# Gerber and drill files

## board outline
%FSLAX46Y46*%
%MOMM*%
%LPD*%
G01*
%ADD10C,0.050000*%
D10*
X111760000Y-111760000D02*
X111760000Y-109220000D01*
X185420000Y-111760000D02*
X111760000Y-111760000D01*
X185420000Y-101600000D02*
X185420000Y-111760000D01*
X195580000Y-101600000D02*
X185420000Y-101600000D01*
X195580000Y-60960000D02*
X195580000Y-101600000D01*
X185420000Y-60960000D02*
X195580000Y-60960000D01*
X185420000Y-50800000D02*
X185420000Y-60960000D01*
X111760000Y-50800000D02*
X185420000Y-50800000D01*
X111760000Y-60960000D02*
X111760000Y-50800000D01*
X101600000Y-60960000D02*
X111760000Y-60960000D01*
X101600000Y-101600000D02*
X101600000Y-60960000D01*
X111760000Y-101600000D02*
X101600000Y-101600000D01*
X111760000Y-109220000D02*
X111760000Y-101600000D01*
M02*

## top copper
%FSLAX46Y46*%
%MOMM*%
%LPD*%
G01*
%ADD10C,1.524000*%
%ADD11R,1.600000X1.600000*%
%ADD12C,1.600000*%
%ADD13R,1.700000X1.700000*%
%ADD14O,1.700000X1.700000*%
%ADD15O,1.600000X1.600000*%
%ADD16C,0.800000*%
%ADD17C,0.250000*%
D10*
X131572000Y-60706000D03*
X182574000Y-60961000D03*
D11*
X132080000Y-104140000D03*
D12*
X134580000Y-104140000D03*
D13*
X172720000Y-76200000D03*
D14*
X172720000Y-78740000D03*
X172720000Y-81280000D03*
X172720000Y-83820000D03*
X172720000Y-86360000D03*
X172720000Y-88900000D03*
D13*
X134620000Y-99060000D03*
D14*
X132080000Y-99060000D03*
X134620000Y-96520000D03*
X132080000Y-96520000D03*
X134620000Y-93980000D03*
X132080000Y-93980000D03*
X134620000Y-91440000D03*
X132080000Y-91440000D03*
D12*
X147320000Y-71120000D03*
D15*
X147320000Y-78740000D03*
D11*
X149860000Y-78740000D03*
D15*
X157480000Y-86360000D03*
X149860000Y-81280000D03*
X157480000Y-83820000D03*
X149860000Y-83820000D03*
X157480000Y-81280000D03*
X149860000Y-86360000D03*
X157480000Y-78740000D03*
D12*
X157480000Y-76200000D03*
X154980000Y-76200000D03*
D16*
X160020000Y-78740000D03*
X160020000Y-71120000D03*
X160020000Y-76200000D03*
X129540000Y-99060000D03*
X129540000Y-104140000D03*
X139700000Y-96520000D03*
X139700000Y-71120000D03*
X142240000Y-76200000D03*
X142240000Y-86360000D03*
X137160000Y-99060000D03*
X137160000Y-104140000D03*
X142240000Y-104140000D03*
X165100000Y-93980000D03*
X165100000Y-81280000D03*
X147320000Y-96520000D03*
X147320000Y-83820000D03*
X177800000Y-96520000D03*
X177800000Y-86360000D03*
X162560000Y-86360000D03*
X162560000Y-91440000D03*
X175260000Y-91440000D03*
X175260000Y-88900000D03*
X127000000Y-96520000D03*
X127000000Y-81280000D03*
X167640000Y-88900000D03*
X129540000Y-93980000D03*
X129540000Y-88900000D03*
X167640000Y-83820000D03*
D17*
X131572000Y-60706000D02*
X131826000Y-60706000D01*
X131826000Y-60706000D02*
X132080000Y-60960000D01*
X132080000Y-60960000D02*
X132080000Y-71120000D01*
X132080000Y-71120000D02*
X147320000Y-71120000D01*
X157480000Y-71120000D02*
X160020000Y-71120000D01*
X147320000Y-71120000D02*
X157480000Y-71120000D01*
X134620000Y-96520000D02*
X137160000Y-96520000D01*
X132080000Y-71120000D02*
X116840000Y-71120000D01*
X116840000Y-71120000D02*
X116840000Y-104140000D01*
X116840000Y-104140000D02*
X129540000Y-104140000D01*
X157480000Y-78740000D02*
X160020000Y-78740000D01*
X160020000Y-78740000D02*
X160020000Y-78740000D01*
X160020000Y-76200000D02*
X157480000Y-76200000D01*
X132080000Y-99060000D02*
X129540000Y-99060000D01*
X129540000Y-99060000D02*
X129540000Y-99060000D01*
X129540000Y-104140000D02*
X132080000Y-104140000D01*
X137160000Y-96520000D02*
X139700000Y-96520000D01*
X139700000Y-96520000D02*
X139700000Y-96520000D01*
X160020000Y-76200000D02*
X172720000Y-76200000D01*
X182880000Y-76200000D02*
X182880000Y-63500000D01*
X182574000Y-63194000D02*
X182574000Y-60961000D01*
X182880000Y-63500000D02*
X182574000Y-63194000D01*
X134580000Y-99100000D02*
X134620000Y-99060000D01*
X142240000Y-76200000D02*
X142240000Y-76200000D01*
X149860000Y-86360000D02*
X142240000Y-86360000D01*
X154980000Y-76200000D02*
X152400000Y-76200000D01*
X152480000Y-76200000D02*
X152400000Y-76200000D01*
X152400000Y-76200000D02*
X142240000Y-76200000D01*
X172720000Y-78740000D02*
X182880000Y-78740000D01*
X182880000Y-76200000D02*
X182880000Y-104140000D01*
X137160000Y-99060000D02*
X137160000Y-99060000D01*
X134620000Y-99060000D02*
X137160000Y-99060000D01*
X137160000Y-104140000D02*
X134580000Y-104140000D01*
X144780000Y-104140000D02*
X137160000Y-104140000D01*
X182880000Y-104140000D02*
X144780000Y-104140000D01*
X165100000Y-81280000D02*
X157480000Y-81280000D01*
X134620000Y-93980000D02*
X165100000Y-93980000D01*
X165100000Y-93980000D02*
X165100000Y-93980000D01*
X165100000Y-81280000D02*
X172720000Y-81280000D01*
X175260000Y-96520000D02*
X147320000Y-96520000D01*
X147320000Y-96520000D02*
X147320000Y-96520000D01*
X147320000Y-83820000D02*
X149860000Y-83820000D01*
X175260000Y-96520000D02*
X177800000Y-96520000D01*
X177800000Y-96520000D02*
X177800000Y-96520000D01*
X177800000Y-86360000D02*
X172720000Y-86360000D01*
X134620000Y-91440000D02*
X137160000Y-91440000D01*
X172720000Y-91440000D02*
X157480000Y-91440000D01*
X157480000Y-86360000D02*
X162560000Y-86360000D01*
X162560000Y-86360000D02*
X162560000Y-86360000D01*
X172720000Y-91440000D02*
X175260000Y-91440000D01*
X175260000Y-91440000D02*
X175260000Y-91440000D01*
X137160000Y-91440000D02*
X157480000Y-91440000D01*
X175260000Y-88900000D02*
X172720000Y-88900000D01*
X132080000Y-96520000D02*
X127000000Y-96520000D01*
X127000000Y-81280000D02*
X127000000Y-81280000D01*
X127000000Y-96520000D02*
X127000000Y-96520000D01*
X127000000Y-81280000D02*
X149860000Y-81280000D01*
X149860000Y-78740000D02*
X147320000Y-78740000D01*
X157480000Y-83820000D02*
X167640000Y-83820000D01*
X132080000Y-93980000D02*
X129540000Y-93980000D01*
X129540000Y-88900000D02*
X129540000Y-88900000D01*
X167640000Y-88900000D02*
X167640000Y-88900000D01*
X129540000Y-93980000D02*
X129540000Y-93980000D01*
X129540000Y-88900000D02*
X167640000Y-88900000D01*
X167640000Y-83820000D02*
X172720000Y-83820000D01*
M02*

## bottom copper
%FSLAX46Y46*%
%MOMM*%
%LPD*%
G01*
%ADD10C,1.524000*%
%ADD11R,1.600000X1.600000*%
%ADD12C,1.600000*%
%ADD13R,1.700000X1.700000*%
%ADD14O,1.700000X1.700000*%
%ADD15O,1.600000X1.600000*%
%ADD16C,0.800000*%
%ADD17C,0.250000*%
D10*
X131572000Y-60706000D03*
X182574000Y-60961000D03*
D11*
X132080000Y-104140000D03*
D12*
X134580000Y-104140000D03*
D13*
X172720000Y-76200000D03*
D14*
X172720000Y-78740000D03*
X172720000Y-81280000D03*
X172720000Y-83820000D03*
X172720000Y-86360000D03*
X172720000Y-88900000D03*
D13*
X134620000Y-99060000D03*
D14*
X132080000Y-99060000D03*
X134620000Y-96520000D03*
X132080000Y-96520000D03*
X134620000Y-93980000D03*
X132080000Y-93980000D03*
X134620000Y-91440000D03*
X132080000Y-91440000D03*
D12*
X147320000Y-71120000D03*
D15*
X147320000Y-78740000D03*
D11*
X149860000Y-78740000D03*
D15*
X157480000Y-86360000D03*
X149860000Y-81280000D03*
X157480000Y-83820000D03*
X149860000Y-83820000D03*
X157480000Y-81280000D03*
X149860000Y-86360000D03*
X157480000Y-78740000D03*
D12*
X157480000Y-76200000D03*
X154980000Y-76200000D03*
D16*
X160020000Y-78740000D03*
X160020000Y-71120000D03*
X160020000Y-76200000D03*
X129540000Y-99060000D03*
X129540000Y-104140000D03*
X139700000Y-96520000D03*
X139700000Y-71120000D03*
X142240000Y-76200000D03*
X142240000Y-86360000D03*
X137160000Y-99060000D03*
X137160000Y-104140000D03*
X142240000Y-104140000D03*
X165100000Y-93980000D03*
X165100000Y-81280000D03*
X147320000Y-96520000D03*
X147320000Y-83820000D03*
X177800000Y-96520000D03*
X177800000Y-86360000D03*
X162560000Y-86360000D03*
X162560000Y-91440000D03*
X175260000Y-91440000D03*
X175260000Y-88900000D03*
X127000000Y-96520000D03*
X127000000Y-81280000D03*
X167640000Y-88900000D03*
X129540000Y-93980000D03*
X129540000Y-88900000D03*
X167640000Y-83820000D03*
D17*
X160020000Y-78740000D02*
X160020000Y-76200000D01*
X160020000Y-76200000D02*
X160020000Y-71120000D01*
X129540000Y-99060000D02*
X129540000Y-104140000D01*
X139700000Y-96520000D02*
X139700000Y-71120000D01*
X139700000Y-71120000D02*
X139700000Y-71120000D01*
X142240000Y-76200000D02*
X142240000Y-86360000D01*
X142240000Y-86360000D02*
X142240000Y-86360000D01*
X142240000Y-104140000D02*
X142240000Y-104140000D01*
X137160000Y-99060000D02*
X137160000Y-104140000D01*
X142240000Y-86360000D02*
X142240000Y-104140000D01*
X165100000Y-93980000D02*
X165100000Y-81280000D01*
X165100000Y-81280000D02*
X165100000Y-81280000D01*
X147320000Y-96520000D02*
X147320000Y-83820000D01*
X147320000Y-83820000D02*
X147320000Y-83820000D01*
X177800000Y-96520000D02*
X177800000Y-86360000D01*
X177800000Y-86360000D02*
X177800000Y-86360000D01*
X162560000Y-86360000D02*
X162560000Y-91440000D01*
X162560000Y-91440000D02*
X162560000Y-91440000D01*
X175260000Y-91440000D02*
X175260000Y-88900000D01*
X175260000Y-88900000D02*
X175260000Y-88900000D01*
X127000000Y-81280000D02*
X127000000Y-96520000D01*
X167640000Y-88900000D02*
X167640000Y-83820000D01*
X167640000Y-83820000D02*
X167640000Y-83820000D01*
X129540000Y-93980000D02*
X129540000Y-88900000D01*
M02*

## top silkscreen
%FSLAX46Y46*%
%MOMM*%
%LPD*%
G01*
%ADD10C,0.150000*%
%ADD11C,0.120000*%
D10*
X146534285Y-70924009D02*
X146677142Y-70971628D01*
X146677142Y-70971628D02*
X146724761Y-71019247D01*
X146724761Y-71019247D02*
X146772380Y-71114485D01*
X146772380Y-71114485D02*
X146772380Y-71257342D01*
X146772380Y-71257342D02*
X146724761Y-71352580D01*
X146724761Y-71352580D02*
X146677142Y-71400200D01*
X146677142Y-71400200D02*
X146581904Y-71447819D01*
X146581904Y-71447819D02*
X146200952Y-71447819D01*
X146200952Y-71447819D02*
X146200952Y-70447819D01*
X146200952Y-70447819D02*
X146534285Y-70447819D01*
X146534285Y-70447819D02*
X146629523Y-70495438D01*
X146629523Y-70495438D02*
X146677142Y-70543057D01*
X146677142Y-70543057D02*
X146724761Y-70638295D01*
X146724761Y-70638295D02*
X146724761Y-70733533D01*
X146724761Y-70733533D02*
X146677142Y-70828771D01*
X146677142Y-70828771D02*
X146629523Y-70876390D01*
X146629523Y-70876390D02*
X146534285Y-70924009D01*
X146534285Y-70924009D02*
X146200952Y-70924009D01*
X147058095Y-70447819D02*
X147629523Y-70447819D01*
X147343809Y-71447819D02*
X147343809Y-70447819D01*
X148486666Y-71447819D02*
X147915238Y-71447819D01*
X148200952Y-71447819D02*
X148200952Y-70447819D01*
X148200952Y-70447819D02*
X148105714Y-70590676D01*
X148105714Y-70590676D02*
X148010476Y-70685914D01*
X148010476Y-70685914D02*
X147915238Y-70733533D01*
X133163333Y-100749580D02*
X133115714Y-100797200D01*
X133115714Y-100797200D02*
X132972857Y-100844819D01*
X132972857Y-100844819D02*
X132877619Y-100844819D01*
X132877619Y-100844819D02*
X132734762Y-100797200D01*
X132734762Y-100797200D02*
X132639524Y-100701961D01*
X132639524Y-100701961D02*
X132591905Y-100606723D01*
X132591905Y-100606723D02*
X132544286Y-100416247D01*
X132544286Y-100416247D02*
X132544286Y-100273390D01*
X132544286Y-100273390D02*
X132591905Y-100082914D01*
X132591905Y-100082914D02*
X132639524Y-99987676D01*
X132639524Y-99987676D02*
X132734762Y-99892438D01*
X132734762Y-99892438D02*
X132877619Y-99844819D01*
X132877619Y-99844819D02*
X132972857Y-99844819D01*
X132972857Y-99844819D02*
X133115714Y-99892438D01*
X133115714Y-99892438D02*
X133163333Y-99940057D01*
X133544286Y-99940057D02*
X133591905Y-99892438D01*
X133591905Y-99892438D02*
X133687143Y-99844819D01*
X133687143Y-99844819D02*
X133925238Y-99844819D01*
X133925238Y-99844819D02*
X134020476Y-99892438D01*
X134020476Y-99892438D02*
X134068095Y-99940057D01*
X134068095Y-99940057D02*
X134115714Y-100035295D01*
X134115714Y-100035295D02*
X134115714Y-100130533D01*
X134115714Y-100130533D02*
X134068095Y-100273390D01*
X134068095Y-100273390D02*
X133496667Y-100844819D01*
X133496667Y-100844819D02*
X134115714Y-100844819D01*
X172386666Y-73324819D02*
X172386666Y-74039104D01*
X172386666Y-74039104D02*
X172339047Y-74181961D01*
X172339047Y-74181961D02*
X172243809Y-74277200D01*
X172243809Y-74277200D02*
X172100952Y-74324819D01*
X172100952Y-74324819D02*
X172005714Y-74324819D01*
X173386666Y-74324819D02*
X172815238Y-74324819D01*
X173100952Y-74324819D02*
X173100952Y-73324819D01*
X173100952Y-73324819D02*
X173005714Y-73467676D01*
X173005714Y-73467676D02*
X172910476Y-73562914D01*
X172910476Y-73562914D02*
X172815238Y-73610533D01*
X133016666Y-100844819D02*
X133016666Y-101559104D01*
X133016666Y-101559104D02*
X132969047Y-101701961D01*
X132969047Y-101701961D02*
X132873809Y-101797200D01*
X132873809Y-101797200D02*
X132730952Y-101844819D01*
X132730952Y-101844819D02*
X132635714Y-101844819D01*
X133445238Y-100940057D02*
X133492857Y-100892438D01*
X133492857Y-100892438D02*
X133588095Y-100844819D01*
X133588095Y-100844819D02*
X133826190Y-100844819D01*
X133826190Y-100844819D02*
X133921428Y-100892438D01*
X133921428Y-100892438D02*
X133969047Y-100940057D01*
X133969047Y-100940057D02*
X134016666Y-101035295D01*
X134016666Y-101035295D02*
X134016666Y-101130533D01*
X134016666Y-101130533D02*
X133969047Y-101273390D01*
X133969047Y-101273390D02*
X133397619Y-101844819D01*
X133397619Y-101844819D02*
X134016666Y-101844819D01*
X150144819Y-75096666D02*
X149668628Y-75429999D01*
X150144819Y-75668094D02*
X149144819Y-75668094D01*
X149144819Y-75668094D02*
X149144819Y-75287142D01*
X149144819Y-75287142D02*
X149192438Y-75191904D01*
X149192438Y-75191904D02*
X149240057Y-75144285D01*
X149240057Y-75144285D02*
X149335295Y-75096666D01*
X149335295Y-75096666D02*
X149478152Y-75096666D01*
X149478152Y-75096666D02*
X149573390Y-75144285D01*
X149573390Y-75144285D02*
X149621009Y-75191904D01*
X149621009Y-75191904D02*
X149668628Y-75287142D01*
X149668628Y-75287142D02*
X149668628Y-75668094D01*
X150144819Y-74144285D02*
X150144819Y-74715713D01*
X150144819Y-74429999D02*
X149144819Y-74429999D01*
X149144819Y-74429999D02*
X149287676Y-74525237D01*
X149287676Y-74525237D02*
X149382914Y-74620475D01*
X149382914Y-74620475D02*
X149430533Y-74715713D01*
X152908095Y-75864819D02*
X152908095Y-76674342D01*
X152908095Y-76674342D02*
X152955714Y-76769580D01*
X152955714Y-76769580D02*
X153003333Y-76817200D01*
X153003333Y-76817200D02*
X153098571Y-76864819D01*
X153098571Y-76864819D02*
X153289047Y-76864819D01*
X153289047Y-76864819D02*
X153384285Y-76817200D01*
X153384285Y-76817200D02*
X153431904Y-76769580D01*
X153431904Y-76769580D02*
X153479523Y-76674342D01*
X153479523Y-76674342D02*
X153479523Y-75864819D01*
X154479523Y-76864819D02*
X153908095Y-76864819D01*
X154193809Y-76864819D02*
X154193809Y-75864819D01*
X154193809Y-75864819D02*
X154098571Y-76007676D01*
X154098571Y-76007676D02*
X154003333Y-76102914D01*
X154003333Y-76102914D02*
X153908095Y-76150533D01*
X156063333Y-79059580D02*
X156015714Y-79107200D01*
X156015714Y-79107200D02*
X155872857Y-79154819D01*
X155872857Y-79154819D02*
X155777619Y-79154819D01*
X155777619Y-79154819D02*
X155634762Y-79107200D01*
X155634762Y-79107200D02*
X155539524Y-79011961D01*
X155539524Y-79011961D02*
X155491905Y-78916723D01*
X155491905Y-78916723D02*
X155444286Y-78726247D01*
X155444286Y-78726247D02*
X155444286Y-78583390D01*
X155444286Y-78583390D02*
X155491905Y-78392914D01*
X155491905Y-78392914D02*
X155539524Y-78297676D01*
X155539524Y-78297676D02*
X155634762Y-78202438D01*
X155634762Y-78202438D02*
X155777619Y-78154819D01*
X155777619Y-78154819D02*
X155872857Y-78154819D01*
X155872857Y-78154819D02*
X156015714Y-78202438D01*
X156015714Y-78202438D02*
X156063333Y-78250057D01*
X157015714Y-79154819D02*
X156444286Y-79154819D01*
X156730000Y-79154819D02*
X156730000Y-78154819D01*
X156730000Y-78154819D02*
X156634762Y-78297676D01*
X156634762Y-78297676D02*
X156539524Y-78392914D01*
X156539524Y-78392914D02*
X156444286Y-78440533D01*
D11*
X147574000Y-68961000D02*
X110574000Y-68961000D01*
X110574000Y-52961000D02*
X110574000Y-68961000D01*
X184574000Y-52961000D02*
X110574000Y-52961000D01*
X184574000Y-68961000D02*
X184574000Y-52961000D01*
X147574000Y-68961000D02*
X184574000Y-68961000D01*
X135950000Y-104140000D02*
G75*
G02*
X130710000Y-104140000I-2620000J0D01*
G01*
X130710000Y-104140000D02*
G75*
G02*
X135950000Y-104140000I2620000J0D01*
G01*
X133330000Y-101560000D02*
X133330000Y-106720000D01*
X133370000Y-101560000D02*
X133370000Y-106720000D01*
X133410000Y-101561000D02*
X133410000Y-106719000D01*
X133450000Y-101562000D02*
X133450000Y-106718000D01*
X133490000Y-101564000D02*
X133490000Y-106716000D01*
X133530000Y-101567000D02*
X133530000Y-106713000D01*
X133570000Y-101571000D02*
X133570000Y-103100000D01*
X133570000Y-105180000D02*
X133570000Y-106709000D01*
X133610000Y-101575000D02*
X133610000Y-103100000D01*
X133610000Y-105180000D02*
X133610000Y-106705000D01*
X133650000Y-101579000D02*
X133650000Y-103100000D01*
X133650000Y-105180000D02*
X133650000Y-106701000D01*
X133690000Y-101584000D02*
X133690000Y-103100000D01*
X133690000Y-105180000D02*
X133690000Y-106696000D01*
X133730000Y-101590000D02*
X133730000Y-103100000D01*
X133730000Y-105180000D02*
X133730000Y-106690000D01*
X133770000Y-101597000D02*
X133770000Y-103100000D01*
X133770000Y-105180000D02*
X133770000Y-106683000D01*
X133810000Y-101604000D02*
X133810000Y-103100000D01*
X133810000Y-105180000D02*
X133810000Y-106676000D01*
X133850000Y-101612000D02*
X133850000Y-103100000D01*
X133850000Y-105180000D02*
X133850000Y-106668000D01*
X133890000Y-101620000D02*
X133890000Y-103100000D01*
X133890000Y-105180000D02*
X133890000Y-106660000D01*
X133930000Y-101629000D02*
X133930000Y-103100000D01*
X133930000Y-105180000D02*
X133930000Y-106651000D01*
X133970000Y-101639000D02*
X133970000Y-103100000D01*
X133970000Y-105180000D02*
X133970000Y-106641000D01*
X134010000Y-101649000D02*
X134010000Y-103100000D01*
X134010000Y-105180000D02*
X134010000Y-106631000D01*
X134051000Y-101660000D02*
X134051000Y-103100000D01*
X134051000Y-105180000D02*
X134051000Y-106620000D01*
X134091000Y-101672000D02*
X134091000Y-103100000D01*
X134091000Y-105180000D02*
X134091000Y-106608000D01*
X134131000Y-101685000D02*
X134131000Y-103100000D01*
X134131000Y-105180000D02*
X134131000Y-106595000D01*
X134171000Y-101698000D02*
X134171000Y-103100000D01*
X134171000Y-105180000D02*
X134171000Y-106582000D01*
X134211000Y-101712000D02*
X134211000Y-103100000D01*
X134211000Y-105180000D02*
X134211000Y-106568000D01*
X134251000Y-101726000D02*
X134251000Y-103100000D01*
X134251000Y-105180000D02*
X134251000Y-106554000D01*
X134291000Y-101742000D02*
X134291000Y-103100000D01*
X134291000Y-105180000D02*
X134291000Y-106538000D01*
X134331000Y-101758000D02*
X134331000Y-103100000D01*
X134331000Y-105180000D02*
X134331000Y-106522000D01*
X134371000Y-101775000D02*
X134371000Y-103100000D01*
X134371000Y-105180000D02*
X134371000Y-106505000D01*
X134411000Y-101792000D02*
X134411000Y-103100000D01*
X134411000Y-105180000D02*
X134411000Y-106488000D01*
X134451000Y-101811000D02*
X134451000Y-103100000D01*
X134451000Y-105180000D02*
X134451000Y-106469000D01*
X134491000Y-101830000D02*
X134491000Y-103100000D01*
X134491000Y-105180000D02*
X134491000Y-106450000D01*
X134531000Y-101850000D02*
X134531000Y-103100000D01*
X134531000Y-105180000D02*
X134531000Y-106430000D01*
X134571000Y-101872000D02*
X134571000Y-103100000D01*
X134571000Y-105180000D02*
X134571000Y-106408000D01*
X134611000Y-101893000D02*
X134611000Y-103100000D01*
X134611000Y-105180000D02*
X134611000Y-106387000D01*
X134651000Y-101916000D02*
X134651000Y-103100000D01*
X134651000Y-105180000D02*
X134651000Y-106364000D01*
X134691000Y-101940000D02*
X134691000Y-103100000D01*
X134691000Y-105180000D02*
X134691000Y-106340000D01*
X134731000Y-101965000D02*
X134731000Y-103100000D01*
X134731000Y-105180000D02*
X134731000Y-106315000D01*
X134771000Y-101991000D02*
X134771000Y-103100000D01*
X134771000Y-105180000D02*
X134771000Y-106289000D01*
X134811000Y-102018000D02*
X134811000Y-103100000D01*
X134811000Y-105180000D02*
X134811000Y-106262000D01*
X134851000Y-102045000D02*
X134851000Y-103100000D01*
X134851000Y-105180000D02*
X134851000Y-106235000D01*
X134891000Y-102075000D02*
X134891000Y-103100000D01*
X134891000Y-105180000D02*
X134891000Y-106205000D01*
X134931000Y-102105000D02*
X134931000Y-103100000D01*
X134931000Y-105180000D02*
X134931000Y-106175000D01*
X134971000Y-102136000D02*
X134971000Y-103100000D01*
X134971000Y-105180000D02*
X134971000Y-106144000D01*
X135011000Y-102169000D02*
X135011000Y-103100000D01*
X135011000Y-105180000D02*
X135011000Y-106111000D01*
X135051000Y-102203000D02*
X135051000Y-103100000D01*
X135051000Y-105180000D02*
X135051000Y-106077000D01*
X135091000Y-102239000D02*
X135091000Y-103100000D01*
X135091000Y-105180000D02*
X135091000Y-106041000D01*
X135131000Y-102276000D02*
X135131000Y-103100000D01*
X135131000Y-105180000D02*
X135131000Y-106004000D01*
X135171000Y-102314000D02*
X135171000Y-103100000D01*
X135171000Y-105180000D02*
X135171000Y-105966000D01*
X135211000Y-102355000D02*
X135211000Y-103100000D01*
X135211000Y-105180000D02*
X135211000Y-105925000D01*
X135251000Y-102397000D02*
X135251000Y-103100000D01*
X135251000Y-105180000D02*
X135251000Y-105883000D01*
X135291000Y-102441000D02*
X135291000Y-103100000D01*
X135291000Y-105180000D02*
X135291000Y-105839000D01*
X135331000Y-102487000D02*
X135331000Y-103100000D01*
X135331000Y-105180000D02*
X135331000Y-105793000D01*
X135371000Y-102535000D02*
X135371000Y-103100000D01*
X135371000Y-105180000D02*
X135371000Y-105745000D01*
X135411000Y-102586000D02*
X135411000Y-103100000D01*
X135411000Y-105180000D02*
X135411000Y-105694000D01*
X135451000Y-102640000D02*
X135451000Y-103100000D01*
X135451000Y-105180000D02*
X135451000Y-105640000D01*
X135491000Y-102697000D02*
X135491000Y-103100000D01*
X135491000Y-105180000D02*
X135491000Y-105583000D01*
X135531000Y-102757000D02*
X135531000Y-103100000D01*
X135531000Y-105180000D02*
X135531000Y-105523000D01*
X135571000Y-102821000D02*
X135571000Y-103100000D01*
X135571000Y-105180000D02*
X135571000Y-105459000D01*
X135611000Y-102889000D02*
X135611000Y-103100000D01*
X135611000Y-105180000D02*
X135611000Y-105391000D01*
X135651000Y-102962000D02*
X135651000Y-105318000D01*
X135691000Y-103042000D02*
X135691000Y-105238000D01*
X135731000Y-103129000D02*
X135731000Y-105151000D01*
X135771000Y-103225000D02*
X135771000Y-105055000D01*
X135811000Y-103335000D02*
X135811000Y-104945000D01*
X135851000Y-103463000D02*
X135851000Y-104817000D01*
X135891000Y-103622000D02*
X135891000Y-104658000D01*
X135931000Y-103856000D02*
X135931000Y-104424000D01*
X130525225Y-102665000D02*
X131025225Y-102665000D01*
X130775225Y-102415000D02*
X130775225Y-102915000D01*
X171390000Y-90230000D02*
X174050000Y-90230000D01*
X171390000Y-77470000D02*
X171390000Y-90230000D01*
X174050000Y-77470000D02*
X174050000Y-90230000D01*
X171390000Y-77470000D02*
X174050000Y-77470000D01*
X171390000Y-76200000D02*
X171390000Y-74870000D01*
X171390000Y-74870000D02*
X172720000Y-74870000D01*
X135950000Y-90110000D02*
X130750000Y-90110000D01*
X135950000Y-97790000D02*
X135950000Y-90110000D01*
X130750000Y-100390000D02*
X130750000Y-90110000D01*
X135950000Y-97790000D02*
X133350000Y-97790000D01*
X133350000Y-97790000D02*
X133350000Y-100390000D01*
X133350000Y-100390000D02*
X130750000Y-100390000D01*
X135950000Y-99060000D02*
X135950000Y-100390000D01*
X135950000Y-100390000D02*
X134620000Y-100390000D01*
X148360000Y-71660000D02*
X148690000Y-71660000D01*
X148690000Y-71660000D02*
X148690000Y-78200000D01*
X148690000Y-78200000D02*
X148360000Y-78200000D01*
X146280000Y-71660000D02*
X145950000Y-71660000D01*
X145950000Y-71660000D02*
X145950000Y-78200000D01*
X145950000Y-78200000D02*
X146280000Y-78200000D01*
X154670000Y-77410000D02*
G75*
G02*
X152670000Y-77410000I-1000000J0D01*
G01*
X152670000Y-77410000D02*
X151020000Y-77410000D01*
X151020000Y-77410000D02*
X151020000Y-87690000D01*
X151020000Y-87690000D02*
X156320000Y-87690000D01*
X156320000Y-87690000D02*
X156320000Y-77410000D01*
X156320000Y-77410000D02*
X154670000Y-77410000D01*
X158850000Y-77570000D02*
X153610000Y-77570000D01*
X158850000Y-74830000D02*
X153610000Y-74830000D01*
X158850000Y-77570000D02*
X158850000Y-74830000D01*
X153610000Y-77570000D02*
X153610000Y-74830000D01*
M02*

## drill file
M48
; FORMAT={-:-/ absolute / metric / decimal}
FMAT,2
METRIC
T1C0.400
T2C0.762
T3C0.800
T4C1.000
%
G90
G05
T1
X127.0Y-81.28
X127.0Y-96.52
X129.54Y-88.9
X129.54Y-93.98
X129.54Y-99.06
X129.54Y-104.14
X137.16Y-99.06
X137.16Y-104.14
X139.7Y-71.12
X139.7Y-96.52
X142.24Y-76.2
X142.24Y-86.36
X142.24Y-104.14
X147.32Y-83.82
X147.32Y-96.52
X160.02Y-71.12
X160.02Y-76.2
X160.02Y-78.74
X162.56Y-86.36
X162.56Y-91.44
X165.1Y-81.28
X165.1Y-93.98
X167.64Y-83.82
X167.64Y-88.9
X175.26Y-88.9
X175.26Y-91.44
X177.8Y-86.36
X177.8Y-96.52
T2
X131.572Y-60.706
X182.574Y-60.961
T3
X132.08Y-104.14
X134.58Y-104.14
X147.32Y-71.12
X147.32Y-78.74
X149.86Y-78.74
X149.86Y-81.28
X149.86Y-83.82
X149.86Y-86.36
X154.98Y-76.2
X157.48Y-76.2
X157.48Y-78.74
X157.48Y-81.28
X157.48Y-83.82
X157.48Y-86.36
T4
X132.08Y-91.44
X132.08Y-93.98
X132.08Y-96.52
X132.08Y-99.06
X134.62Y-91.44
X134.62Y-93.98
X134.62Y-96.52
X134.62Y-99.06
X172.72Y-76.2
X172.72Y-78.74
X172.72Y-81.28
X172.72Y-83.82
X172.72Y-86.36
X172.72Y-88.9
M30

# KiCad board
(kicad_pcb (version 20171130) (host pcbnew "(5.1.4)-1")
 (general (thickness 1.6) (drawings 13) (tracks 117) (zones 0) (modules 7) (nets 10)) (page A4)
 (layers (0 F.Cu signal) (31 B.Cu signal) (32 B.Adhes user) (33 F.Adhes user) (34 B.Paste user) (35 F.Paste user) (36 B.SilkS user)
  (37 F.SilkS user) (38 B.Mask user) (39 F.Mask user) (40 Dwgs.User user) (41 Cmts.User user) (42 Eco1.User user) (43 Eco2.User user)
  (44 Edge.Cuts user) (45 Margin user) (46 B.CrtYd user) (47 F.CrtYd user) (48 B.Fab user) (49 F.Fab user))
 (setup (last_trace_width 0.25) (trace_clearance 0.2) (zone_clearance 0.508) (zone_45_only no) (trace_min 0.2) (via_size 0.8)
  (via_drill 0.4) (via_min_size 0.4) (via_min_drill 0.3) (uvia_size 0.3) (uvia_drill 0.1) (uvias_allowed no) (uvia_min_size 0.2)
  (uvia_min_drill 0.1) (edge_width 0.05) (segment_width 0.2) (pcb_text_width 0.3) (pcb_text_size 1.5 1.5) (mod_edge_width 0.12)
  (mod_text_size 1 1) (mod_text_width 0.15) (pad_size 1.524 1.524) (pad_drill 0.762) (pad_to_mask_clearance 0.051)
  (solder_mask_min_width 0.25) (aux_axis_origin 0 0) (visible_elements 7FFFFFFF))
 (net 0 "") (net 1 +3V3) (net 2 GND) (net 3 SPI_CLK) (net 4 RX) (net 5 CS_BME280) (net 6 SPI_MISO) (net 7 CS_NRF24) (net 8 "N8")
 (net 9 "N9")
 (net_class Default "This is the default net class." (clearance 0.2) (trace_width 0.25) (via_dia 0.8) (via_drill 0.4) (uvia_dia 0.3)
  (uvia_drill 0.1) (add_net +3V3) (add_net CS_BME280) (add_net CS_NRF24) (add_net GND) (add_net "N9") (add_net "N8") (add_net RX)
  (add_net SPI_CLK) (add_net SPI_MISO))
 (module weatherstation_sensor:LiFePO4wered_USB (layer F.Cu) (at 147.32 60.96 180)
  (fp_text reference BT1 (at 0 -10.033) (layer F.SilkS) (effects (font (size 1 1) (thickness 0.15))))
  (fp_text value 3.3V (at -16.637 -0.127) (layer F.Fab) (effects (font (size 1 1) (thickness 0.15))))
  (fp_line (start -0.254 -8.001) (end 36.746 -8.001) (layer F.SilkS) (width 0.12))
  (fp_line (start 36.746 7.999) (end 36.746 -8.001) (layer F.SilkS) (width 0.12))
  (fp_line (start -37.254 7.999) (end 36.746 7.999) (layer F.SilkS) (width 0.12))
  (fp_line (start -37.254 -8.001) (end -37.254 7.999) (layer F.SilkS) (width 0.12))
  (fp_line (start -0.254 -8.001) (end -37.254 -8.001) (layer F.SilkS) (width 0.12))
  (pad 1 thru_hole circle (at 15.748 0.254 180) (size 1.524 1.524) (drill 0.762) (layers *.Cu *.Mask) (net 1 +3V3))
  (pad 2 thru_hole circle (at -35.254 -0.001 180) (size 1.524 1.524) (drill 0.762) (layers *.Cu *.Mask) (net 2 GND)))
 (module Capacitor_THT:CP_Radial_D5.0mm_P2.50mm (layer F.Cu) (at 132.08 104.14)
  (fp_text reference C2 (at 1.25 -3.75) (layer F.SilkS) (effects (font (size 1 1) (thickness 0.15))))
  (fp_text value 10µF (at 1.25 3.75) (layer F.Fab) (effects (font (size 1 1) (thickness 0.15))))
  (fp_circle (center 1.25 0) (end 3.87 0) (layer F.SilkS) (width 0.12))
  (fp_line (start 1.25 -2.58) (end 1.25 2.58) (layer F.SilkS) (width 0.12))
  (fp_line (start 1.29 -2.58) (end 1.29 2.58) (layer F.SilkS) (width 0.12))
  (fp_line (start 1.33 -2.579) (end 1.33 2.579) (layer F.SilkS) (width 0.12))
  (fp_line (start 1.37 -2.578) (end 1.37 2.578) (layer F.SilkS) (width 0.12))
  (fp_line (start 1.41 -2.576) (end 1.41 2.576) (layer F.SilkS) (width 0.12))
  (fp_line (start 1.45 -2.573) (end 1.45 2.573) (layer F.SilkS) (width 0.12))
  (fp_line (start 1.49 -2.569) (end 1.49 -1.04) (layer F.SilkS) (width 0.12))
  (fp_line (start 1.49 1.04) (end 1.49 2.569) (layer F.SilkS) (width 0.12))
  (fp_line (start 1.53 -2.565) (end 1.53 -1.04) (layer F.SilkS) (width 0.12))
  (fp_line (start 1.53 1.04) (end 1.53 2.565) (layer F.SilkS) (width 0.12))
  (fp_line (start 1.57 -2.561) (end 1.57 -1.04) (layer F.SilkS) (width 0.12))
  (fp_line (start 1.57 1.04) (end 1.57 2.561) (layer F.SilkS) (width 0.12))
  (fp_line (start 1.61 -2.556) (end 1.61 -1.04) (layer F.SilkS) (width 0.12))
  (fp_line (start 1.61 1.04) (end 1.61 2.556) (layer F.SilkS) (width 0.12))
  (fp_line (start 1.65 -2.55) (end 1.65 -1.04) (layer F.SilkS) (width 0.12))
  (fp_line (start 1.65 1.04) (end 1.65 2.55) (layer F.SilkS) (width 0.12))
  (fp_line (start 1.69 -2.543) (end 1.69 -1.04) (layer F.SilkS) (width 0.12))
  (fp_line (start 1.69 1.04) (end 1.69 2.543) (layer F.SilkS) (width 0.12))
  (fp_line (start 1.73 -2.536) (end 1.73 -1.04) (layer F.SilkS) (width 0.12))
  (fp_line (start 1.73 1.04) (end 1.73 2.536) (layer F.SilkS) (width 0.12))
  (fp_line (start 1.77 -2.528) (end 1.77 -1.04) (layer F.SilkS) (width 0.12))
  (fp_line (start 1.77 1.04) (end 1.77 2.528) (layer F.SilkS) (width 0.12))
  (fp_line (start 1.81 -2.52) (end 1.81 -1.04) (layer F.SilkS) (width 0.12))
  (fp_line (start 1.81 1.04) (end 1.81 2.52) (layer F.SilkS) (width 0.12))
  (fp_line (start 1.85 -2.511) (end 1.85 -1.04) (layer F.SilkS) (width 0.12))
  (fp_line (start 1.85 1.04) (end 1.85 2.511) (layer F.SilkS) (width 0.12))
  (fp_line (start 1.89 -2.501) (end 1.89 -1.04) (layer F.SilkS) (width 0.12))
  (fp_line (start 1.89 1.04) (end 1.89 2.501) (layer F.SilkS) (width 0.12))
  (fp_line (start 1.93 -2.491) (end 1.93 -1.04) (layer F.SilkS) (width 0.12))
  (fp_line (start 1.93 1.04) (end 1.93 2.491) (layer F.SilkS) (width 0.12))
  (fp_line (start 1.971 -2.48) (end 1.971 -1.04) (layer F.SilkS) (width 0.12))
  (fp_line (start 1.971 1.04) (end 1.971 2.48) (layer F.SilkS) (width 0.12))
  (fp_line (start 2.011 -2.468) (end 2.011 -1.04) (layer F.SilkS) (width 0.12))
  (fp_line (start 2.011 1.04) (end 2.011 2.468) (layer F.SilkS) (width 0.12))
  (fp_line (start 2.051 -2.455) (end 2.051 -1.04) (layer F.SilkS) (width 0.12))
  (fp_line (start 2.051 1.04) (end 2.051 2.455) (layer F.SilkS) (width 0.12))
  (fp_line (start 2.091 -2.442) (end 2.091 -1.04) (layer F.SilkS) (width 0.12))
  (fp_line (start 2.091 1.04) (end 2.091 2.442) (layer F.SilkS) (width 0.12))
  (fp_line (start 2.131 -2.428) (end 2.131 -1.04) (layer F.SilkS) (width 0.12))
  (fp_line (start 2.131 1.04) (end 2.131 2.428) (layer F.SilkS) (width 0.12))
  (fp_line (start 2.171 -2.414) (end 2.171 -1.04) (layer F.SilkS) (width 0.12))
  (fp_line (start 2.171 1.04) (end 2.171 2.414) (layer F.SilkS) (width 0.12))
  (fp_line (start 2.211 -2.398) (end 2.211 -1.04) (layer F.SilkS) (width 0.12))
  (fp_line (start 2.211 1.04) (end 2.211 2.398) (layer F.SilkS) (width 0.12))
  (fp_line (start 2.251 -2.382) (end 2.251 -1.04) (layer F.SilkS) (width 0.12))
  (fp_line (start 2.251 1.04) (end 2.251 2.382) (layer F.SilkS) (width 0.12))
  (fp_line (start 2.291 -2.365) (end 2.291 -1.04) (layer F.SilkS) (width 0.12))
  (fp_line (start 2.291 1.04) (end 2.291 2.365) (layer F.SilkS) (width 0.12))
  (fp_line (start 2.331 -2.348) (end 2.331 -1.04) (layer F.SilkS) (width 0.12))
  (fp_line (start 2.331 1.04) (end 2.331 2.348) (layer F.SilkS) (width 0.12))
  (fp_line (start 2.371 -2.329) (end 2.371 -1.04) (layer F.SilkS) (width 0.12))
  (fp_line (start 2.371 1.04) (end 2.371 2.329) (layer F.SilkS) (width 0.12))
  (fp_line (start 2.411 -2.31) (end 2.411 -1.04) (layer F.SilkS) (width 0.12))
  (fp_line (start 2.411 1.04) (end 2.411 2.31) (layer F.SilkS) (width 0.12))
  (fp_line (start 2.451 -2.29) (end 2.451 -1.04) (layer F.SilkS) (width 0.12))
  (fp_line (start 2.451 1.04) (end 2.451 2.29) (layer F.SilkS) (width 0.12))
  (fp_line (start 2.491 -2.268) (end 2.491 -1.04) (layer F.SilkS) (width 0.12))
  (fp_line (start 2.491 1.04) (end 2.491 2.268) (layer F.SilkS) (width 0.12))
  (fp_line (start 2.531 -2.247) (end 2.531 -1.04) (layer F.SilkS) (width 0.12))
  (fp_line (start 2.531 1.04) (end 2.531 2.247) (layer F.SilkS) (width 0.12))
  (fp_line (start 2.571 -2.224) (end 2.571 -1.04) (layer F.SilkS) (width 0.12))
  (fp_line (start 2.571 1.04) (end 2.571 2.224) (layer F.SilkS) (width 0.12))
  (fp_line (start 2.611 -2.2) (end 2.611 -1.04) (layer F.SilkS) (width 0.12))
  (fp_line (start 2.611 1.04) (end 2.611 2.2) (layer F.SilkS) (width 0.12))
  (fp_line (start 2.651 -2.175) (end 2.651 -1.04) (layer F.SilkS) (width 0.12))
  (fp_line (start 2.651 1.04) (end 2.651 2.175) (layer F.SilkS) (width 0.12))
  (fp_line (start 2.691 -2.149) (end 2.691 -1.04) (layer F.SilkS) (width 0.12))
  (fp_line (start 2.691 1.04) (end 2.691 2.149) (layer F.SilkS) (width 0.12))
  (fp_line (start 2.731 -2.122) (end 2.731 -1.04) (layer F.SilkS) (width 0.12))
  (fp_line (start 2.731 1.04) (end 2.731 2.122) (layer F.SilkS) (width 0.12))
  (fp_line (start 2.771 -2.095) (end 2.771 -1.04) (layer F.SilkS) (width 0.12))
  (fp_line (start 2.771 1.04) (end 2.771 2.095) (layer F.SilkS) (width 0.12))
  (fp_line (start 2.811 -2.065) (end 2.811 -1.04) (layer F.SilkS) (width 0.12))
  (fp_line (start 2.811 1.04) (end 2.811 2.065) (layer F.SilkS) (width 0.12))
  (fp_line (start 2.851 -2.035) (end 2.851 -1.04) (layer F.SilkS) (width 0.12))
  (fp_line (start 2.851 1.04) (end 2.851 2.035) (layer F.SilkS) (width 0.12))
  (fp_line (start 2.891 -2.004) (end 2.891 -1.04) (layer F.SilkS) (width 0.12))
  (fp_line (start 2.891 1.04) (end 2.891 2.004) (layer F.SilkS) (width 0.12))
  (fp_line (start 2.931 -1.971) (end 2.931 -1.04) (layer F.SilkS) (width 0.12))
  (fp_line (start 2.931 1.04) (end 2.931 1.971) (layer F.SilkS) (width 0.12))
  (fp_line (start 2.971 -1.937) (end 2.971 -1.04) (layer F.SilkS) (width 0.12))
  (fp_line (start 2.971 1.04) (end 2.971 1.937) (layer F.SilkS) (width 0.12))
  (fp_line (start 3.011 -1.901) (end 3.011 -1.04) (layer F.SilkS) (width 0.12))
  (fp_line (start 3.011 1.04) (end 3.011 1.901) (layer F.SilkS) (width 0.12))
  (fp_line (start 3.051 -1.864) (end 3.051 -1.04) (layer F.SilkS) (width 0.12))
  (fp_line (start 3.051 1.04) (end 3.051 1.864) (layer F.SilkS) (width 0.12))
  (fp_line (start 3.091 -1.826) (end 3.091 -1.04) (layer F.SilkS) (width 0.12))
  (fp_line (start 3.091 1.04) (end 3.091 1.826) (layer F.SilkS) (width 0.12))
  (fp_line (start 3.131 -1.785) (end 3.131 -1.04) (layer F.SilkS) (width 0.12))
  (fp_line (start 3.131 1.04) (end 3.131 1.785) (layer F.SilkS) (width 0.12))
  (fp_line (start 3.171 -1.743) (end 3.171 -1.04) (layer F.SilkS) (width 0.12))
  (fp_line (start 3.171 1.04) (end 3.171 1.743) (layer F.SilkS) (width 0.12))
  (fp_line (start 3.211 -1.699) (end 3.211 -1.04) (layer F.SilkS) (width 0.12))
  (fp_line (start 3.211 1.04) (end 3.211 1.699) (layer F.SilkS) (width 0.12))
  (fp_line (start 3.251 -1.653) (end 3.251 -1.04) (layer F.SilkS) (width 0.12))
  (fp_line (start 3.251 1.04) (end 3.251 1.653) (layer F.SilkS) (width 0.12))
  (fp_line (start 3.291 -1.605) (end 3.291 -1.04) (layer F.SilkS) (width 0.12))
  (fp_line (start 3.291 1.04) (end 3.291 1.605) (layer F.SilkS) (width 0.12))
  (fp_line (start 3.331 -1.554) (end 3.331 -1.04) (layer F.SilkS) (width 0.12))
  (fp_line (start 3.331 1.04) (end 3.331 1.554) (layer F.SilkS) (width 0.12))
  (fp_line (start 3.371 -1.5) (end 3.371 -1.04) (layer F.SilkS) (width 0.12))
  (fp_line (start 3.371 1.04) (end 3.371 1.5) (layer F.SilkS) (width 0.12))
  (fp_line (start 3.411 -1.443) (end 3.411 -1.04) (layer F.SilkS) (width 0.12))
  (fp_line (start 3.411 1.04) (end 3.411 1.443) (layer F.SilkS) (width 0.12))
  (fp_line (start 3.451 -1.383) (end 3.451 -1.04) (layer F.SilkS) (width 0.12))
  (fp_line (start 3.451 1.04) (end 3.451 1.383) (layer F.SilkS) (width 0.12))
  (fp_line (start 3.491 -1.319) (end 3.491 -1.04) (layer F.SilkS) (width 0.12))
  (fp_line (start 3.491 1.04) (end 3.491 1.319) (layer F.SilkS) (width 0.12))
  (fp_line (start 3.531 -1.251) (end 3.531 -1.04) (layer F.SilkS) (width 0.12))
  (fp_line (start 3.531 1.04) (end 3.531 1.251) (layer F.SilkS) (width 0.12))
  (fp_line (start 3.571 -1.178) (end 3.571 1.178) (layer F.SilkS) (width 0.12))
  (fp_line (start 3.611 -1.098) (end 3.611 1.098) (layer F.SilkS) (width 0.12))
  (fp_line (start 3.651 -1.011) (end 3.651 1.011) (layer F.SilkS) (width 0.12))
  (fp_line (start 3.691 -0.915) (end 3.691 0.915) (layer F.SilkS) (width 0.12))
  (fp_line (start 3.731 -0.805) (end 3.731 0.805) (layer F.SilkS) (width 0.12))
  (fp_line (start 3.771 -0.677) (end 3.771 0.677) (layer F.SilkS) (width 0.12))
  (fp_line (start 3.811 -0.518) (end 3.811 0.518) (layer F.SilkS) (width 0.12))
  (fp_line (start 3.851 -0.284) (end 3.851 0.284) (layer F.SilkS) (width 0.12))
  (fp_line (start -1.554775 -1.475) (end -1.054775 -1.475) (layer F.SilkS) (width 0.12))
  (fp_line (start -1.304775 -1.725) (end -1.304775 -1.225) (layer F.SilkS) (width 0.12))
  (pad 1 thru_hole rect (at 0 0) (size 1.6 1.6) (drill 0.8) (layers *.Cu *.Mask) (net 1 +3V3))
  (pad 2 thru_hole circle (at 2.5 0) (size 1.6 1.6) (drill 0.8) (layers *.Cu *.Mask) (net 2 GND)))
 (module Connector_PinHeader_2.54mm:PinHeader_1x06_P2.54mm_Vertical (layer F.Cu) (at 172.72 76.2)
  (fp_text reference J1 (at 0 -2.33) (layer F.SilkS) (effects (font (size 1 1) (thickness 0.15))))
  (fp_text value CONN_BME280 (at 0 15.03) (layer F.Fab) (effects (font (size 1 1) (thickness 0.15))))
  (fp_line (start -1.33 14.03) (end 1.33 14.03) (layer F.SilkS) (width 0.12))
  (fp_line (start -1.33 1.27) (end -1.33 14.03) (layer F.SilkS) (width 0.12))
  (fp_line (start 1.33 1.27) (end 1.33 14.03) (layer F.SilkS) (width 0.12))
  (fp_line (start -1.33 1.27) (end 1.33 1.27) (layer F.SilkS) (width 0.12))
  (fp_line (start -1.33 0) (end -1.33 -1.33) (layer F.SilkS) (width 0.12))
  (fp_line (start -1.33 -1.33) (end 0 -1.33) (layer F.SilkS) (width 0.12))
  (pad 1 thru_hole rect (at 0 0) (size 1.7 1.7) (drill 1) (layers *.Cu *.Mask) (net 1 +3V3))
  (pad 2 thru_hole oval (at 0 2.54) (size 1.7 1.7) (drill 1) (layers *.Cu *.Mask) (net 2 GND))
  (pad 3 thru_hole oval (at 0 5.08) (size 1.7 1.7) (drill 1) (layers *.Cu *.Mask) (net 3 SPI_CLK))
  (pad 4 thru_hole oval (at 0 7.62) (size 1.7 1.7) (drill 1) (layers *.Cu *.Mask) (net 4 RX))
  (pad 5 thru_hole oval (at 0 10.16) (size 1.7 1.7) (drill 1) (layers *.Cu *.Mask) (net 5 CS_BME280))
  (pad 6 thru_hole oval (at 0 12.7) (size 1.7 1.7) (drill 1) (layers *.Cu *.Mask) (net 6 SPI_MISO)))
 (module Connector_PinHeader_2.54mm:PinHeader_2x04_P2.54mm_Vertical (layer F.Cu) (at 134.62 99.06 180)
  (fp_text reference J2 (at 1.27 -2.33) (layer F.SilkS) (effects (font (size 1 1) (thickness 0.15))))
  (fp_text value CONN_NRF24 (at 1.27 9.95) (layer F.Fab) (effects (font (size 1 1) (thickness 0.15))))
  (fp_line (start -1.33 8.95) (end 3.87 8.95) (layer F.SilkS) (width 0.12))
  (fp_line (start -1.33 1.27) (end -1.33 8.95) (layer F.SilkS) (width 0.12))
  (fp_line (start 3.87 -1.33) (end 3.87 8.95) (layer F.SilkS) (width 0.12))
  (fp_line (start -1.33 1.27) (end 1.27 1.27) (layer F.SilkS) (width 0.12))
  (fp_line (start 1.27 1.27) (end 1.27 -1.33) (layer F.SilkS) (width 0.12))
  (fp_line (start 1.27 -1.33) (end 3.87 -1.33) (layer F.SilkS) (width 0.12))
  (fp_line (start -1.33 0) (end -1.33 -1.33) (layer F.SilkS) (width 0.12))
  (fp_line (start -1.33 -1.33) (end 0 -1.33) (layer F.SilkS) (width 0.12))
  (pad 1 thru_hole rect (at 0 0 180) (size 1.7 1.7) (drill 1) (layers *.Cu *.Mask) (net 2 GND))
  (pad 2 thru_hole oval (at 2.54 0 180) (size 1.7 1.7) (drill 1) (layers *.Cu *.Mask) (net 1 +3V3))
  (pad 3 thru_hole oval (at 0 2.54 180) (size 1.7 1.7) (drill 1) (layers *.Cu *.Mask) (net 1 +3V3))
  (pad 4 thru_hole oval (at 2.54 2.54 180) (size 1.7 1.7) (drill 1) (layers *.Cu *.Mask) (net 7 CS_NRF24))
  (pad 5 thru_hole oval (at 0 5.08 180) (size 1.7 1.7) (drill 1) (layers *.Cu *.Mask) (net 3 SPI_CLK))
  (pad 6 thru_hole oval (at 2.54 5.08 180) (size 1.7 1.7) (drill 1) (layers *.Cu *.Mask) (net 4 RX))
  (pad 7 thru_hole oval (at 0 7.62 180) (size 1.7 1.7) (drill 1) (layers *.Cu *.Mask) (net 6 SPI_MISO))
  (pad 8 thru_hole oval (at 2.54 7.62 180) (size 1.7 1.7) (drill 1) (layers *.Cu *.Mask) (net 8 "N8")))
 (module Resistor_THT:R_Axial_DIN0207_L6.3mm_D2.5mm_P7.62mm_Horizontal (layer F.Cu) (at 147.32 71.12 270)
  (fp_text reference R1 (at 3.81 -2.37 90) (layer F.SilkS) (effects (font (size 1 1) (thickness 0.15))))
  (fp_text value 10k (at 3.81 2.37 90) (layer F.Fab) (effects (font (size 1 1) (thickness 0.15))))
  (fp_line (start 0.54 -1.04) (end 0.54 -1.37) (layer F.SilkS) (width 0.12))
  (fp_line (start 0.54 -1.37) (end 7.08 -1.37) (layer F.SilkS) (width 0.12))
  (fp_line (start 7.08 -1.37) (end 7.08 -1.04) (layer F.SilkS) (width 0.12))
  (fp_line (start 0.54 1.04) (end 0.54 1.37) (layer F.SilkS) (width 0.12))
  (fp_line (start 0.54 1.37) (end 7.08 1.37) (layer F.SilkS) (width 0.12))
  (fp_line (start 7.08 1.37) (end 7.08 1.04) (layer F.SilkS) (width 0.12))
  (pad 1 thru_hole circle (at 0 0 270) (size 1.6 1.6) (drill 0.8) (layers *.Cu *.Mask) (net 1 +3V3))
  (pad 2 thru_hole oval (at 7.62 0 270) (size 1.6 1.6) (drill 0.8) (layers *.Cu *.Mask) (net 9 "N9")))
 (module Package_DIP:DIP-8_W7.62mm (layer F.Cu) (at 149.86 78.74)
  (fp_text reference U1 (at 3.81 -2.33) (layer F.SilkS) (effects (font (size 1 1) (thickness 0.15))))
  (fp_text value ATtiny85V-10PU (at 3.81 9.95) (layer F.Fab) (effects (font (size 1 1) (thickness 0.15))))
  (fp_arc (start 3.81 -1.33) (end 2.81 -1.33) (angle -180) (layer F.SilkS) (width 0.12))
  (fp_line (start 2.81 -1.33) (end 1.16 -1.33) (layer F.SilkS) (width 0.12))
  (fp_line (start 1.16 -1.33) (end 1.16 8.95) (layer F.SilkS) (width 0.12))
  (fp_line (start 1.16 8.95) (end 6.46 8.95) (layer F.SilkS) (width 0.12))
  (fp_line (start 6.46 8.95) (end 6.46 -1.33) (layer F.SilkS) (width 0.12))
  (fp_line (start 6.46 -1.33) (end 4.81 -1.33) (layer F.SilkS) (width 0.12))
  (pad 1 thru_hole rect (at 0 0) (size 1.6 1.6) (drill 0.8) (layers *.Cu *.Mask) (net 9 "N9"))
  (pad 5 thru_hole oval (at 7.62 7.62) (size 1.6 1.6) (drill 0.8) (layers *.Cu *.Mask) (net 6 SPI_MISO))
  (pad 2 thru_hole oval (at 0 2.54) (size 1.6 1.6) (drill 0.8) (layers *.Cu *.Mask) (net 7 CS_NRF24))
  (pad 6 thru_hole oval (at 7.62 5.08) (size 1.6 1.6) (drill 0.8) (layers *.Cu *.Mask) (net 4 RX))
  (pad 3 thru_hole oval (at 0 5.08) (size 1.6 1.6) (drill 0.8) (layers *.Cu *.Mask) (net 5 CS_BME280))
  (pad 7 thru_hole oval (at 7.62 2.54) (size 1.6 1.6) (drill 0.8) (layers *.Cu *.Mask) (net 3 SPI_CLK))
  (pad 4 thru_hole oval (at 0 7.62) (size 1.6 1.6) (drill 0.8) (layers *.Cu *.Mask) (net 2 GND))
  (pad 8 thru_hole oval (at 7.62 0) (size 1.6 1.6) (drill 0.8) (layers *.Cu *.Mask) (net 1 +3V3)))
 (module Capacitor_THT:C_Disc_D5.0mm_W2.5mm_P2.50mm (layer F.Cu) (at 157.48 76.2 180)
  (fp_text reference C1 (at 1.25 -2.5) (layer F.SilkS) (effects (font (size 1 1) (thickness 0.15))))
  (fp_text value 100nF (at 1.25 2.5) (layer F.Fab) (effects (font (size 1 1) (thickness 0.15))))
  (fp_line (start -1.37 -1.37) (end 3.87 -1.37) (layer F.SilkS) (width 0.12))
  (fp_line (start -1.37 1.37) (end 3.87 1.37) (layer F.SilkS) (width 0.12))
  (fp_line (start -1.37 -1.37) (end -1.37 1.37) (layer F.SilkS) (width 0.12))
  (fp_line (start 3.87 -1.37) (end 3.87 1.37) (layer F.SilkS) (width 0.12))
  (pad 1 thru_hole circle (at 0 0 180) (size 1.6 1.6) (drill 0.8) (layers *.Cu *.Mask) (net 1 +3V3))
  (pad 2 thru_hole circle (at 2.5 0 180) (size 1.6 1.6) (drill 0.8) (layers *.Cu *.Mask) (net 2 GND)))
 (gr_line (start 111.76 111.76) (end 111.76 109.22) (layer Edge.Cuts) (width 0.05))
 (gr_line (start 185.42 111.76) (end 111.76 111.76) (layer Edge.Cuts) (width 0.05))
 (gr_line (start 185.42 101.6) (end 185.42 111.76) (layer Edge.Cuts) (width 0.05))
 (gr_line (start 195.58 101.6) (end 185.42 101.6) (layer Edge.Cuts) (width 0.05))
 (gr_line (start 195.58 60.96) (end 195.58 101.6) (layer Edge.Cuts) (width 0.05))
 (gr_line (start 185.42 60.96) (end 195.58 60.96) (layer Edge.Cuts) (width 0.05))
 (gr_line (start 185.42 50.8) (end 185.42 60.96) (layer Edge.Cuts) (width 0.05))
 (gr_line (start 111.76 50.8) (end 185.42 50.8) (layer Edge.Cuts) (width 0.05))
 (gr_line (start 111.76 60.96) (end 111.76 50.8) (layer Edge.Cuts) (width 0.05))
 (gr_line (start 101.6 60.96) (end 111.76 60.96) (layer Edge.Cuts) (width 0.05))
 (gr_line (start 101.6 101.6) (end 101.6 60.96) (layer Edge.Cuts) (width 0.05))
 (gr_line (start 111.76 101.6) (end 101.6 101.6) (layer Edge.Cuts) (width 0.05))
 (gr_line (start 111.76 109.22) (end 111.76 101.6) (layer Edge.Cuts) (width 0.05))
 (segment (start 131.572 60.706) (end 131.826 60.706) (width 0.25) (layer F.Cu) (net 1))
 (segment (start 131.826 60.706) (end 132.08 60.96) (width 0.25) (layer F.Cu) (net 1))
 (segment (start 132.08 60.96) (end 132.08 71.12) (width 0.25) (layer F.Cu) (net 1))
 (segment (start 132.08 71.12) (end 147.32 71.12) (width 0.25) (layer F.Cu) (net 1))
 (segment (start 157.48 71.12) (end 160.02 71.12) (width 0.25) (layer F.Cu) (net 1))
 (segment (start 147.32 71.12) (end 157.48 71.12) (width 0.25) (layer F.Cu) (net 1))
 (segment (start 134.62 96.52) (end 137.16 96.52) (width 0.25) (layer F.Cu) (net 1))
 (segment (start 132.08 71.12) (end 116.84 71.12) (width 0.25) (layer F.Cu) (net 1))
 (segment (start 116.84 71.12) (end 116.84 104.14) (width 0.25) (layer F.Cu) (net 1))
 (segment (start 116.84 104.14) (end 129.54 104.14) (width 0.25) (layer F.Cu) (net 1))
 (segment (start 157.48 78.74) (end 160.02 78.74) (width 0.25) (layer F.Cu) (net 1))
 (segment (start 160.02 78.74) (end 160.02 78.74) (width 0.25) (layer F.Cu) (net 1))
 (via (at 160.02 78.74) (size 0.8) (drill 0.4) (layers F.Cu B.Cu) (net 1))
 (via (at 160.02 71.12) (size 0.8) (drill 0.4) (layers F.Cu B.Cu) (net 1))
 (segment (start 160.02 78.74) (end 160.02 76.2) (width 0.25) (layer B.Cu) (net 1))
 (segment (start 160.02 76.2) (end 160.02 71.12) (width 0.25) (layer B.Cu) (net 1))
 (via (at 160.02 76.2) (size 0.8) (drill 0.4) (layers F.Cu B.Cu) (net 1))
 (segment (start 160.02 76.2) (end 157.48 76.2) (width 0.25) (layer F.Cu) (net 1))
 (segment (start 132.08 99.06) (end 129.54 99.06) (width 0.25) (layer F.Cu) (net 1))
 (segment (start 129.54 99.06) (end 129.54 99.06) (width 0.25) (layer F.Cu) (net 1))
 (via (at 129.54 99.06) (size 0.8) (drill 0.4) (layers F.Cu B.Cu) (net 1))
 (segment (start 129.54 104.14) (end 132.08 104.14) (width 0.25) (layer F.Cu) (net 1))
 (via (at 129.54 104.14) (size 0.8) (drill 0.4) (layers F.Cu B.Cu) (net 1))
 (segment (start 129.54 99.06) (end 129.54 104.14) (width 0.25) (layer B.Cu) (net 1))
 (segment (start 137.16 96.52) (end 139.7 96.52) (width 0.25) (layer F.Cu) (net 1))
 (segment (start 139.7 96.52) (end 139.7 96.52) (width 0.25) (layer F.Cu) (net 1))
 (via (at 139.7 96.52) (size 0.8) (drill 0.4) (layers F.Cu B.Cu) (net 1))
 (segment (start 139.7 96.52) (end 139.7 71.12) (width 0.25) (layer B.Cu) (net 1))
 (segment (start 139.7 71.12) (end 139.7 71.12) (width 0.25) (layer B.Cu) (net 1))
 (via (at 139.7 71.12) (size 0.8) (drill 0.4) (layers F.Cu B.Cu) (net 1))
 (segment (start 160.02 76.2) (end 172.72 76.2) (width 0.25) (layer F.Cu) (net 1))
 (segment (start 182.88 76.2) (end 182.88 63.5) (width 0.25) (layer F.Cu) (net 2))
 (segment (start 182.574 63.194) (end 182.574 60.961) (width 0.25) (layer F.Cu) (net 2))
 (segment (start 182.88 63.5) (end 182.574 63.194) (width 0.25) (layer F.Cu) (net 2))
 (segment (start 134.58 99.1) (end 134.62 99.06) (width 0.25) (layer F.Cu) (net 2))
 (segment (start 142.24 76.2) (end 142.24 76.2) (width 0.25) (layer F.Cu) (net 2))
 (via (at 142.24 76.2) (size 0.8) (drill 0.4) (layers F.Cu B.Cu) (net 2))
 (segment (start 142.24 76.2) (end 142.24 86.36) (width 0.25) (layer B.Cu) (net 2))
 (segment (start 142.24 86.36) (end 142.24 86.36) (width 0.25) (layer B.Cu) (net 2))
 (via (at 142.24 86.36) (size 0.8) (drill 0.4) (layers F.Cu B.Cu) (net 2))
 (segment (start 149.86 86.36) (end 142.24 86.36) (width 0.25) (layer F.Cu) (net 2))
 (segment (start 154.98 76.2) (end 152.4 76.2) (width 0.25) (layer F.Cu) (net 2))
 (segment (start 152.48 76.2) (end 152.4 76.2) (width 0.25) (layer F.Cu) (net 2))
 (segment (start 152.4 76.2) (end 142.24 76.2) (width 0.25) (layer F.Cu) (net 2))
 (segment (start 172.72 78.74) (end 182.88 78.74) (width 0.25) (layer F.Cu) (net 2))
 (segment (start 182.88 76.2) (end 182.88 104.14) (width 0.25) (layer F.Cu) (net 2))
 (segment (start 137.16 99.06) (end 137.16 99.06) (width 0.25) (layer F.Cu) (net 2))
 (segment (start 134.62 99.06) (end 137.16 99.06) (width 0.25) (layer F.Cu) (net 2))
 (via (at 137.16 99.06) (size 0.8) (drill 0.4) (layers F.Cu B.Cu) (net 2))
 (segment (start 137.16 104.14) (end 134.58 104.14) (width 0.25) (layer F.Cu) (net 2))
 (via (at 137.16 104.14) (size 0.8) (drill 0.4) (layers F.Cu B.Cu) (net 2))
 (segment (start 142.24 104.14) (end 142.24 104.14) (width 0.25) (layer B.Cu) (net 2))
 (segment (start 137.16 99.06) (end 137.16 104.14) (width 0.25) (layer B.Cu) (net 2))
 (segment (start 142.24 86.36) (end 142.24 104.14) (width 0.25) (layer B.Cu) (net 2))
 (via (at 142.24 104.14) (size 0.8) (drill 0.4) (layers F.Cu B.Cu) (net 2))
 (segment (start 144.78 104.14) (end 137.16 104.14) (width 0.25) (layer F.Cu) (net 2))
 (segment (start 182.88 104.14) (end 144.78 104.14) (width 0.25) (layer F.Cu) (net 2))
 (segment (start 165.1 81.28) (end 157.48 81.28) (width 0.25) (layer F.Cu) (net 3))
 (segment (start 134.62 93.98) (end 165.1 93.98) (width 0.25) (layer F.Cu) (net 3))
 (segment (start 165.1 93.98) (end 165.1 93.98) (width 0.25) (layer F.Cu) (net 3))
 (via (at 165.1 93.98) (size 0.8) (drill 0.4) (layers F.Cu B.Cu) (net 3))
 (segment (start 165.1 93.98) (end 165.1 81.28) (width 0.25) (layer B.Cu) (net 3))
 (segment (start 165.1 81.28) (end 165.1 81.28) (width 0.25) (layer B.Cu) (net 3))
 (via (at 165.1 81.28) (size 0.8) (drill 0.4) (layers F.Cu B.Cu) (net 3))
 (segment (start 165.1 81.28) (end 172.72 81.28) (width 0.25) (layer F.Cu) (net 3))
 (segment (start 175.26 96.52) (end 147.32 96.52) (width 0.25) (layer F.Cu) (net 5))
 (segment (start 147.32 96.52) (end 147.32 96.52) (width 0.25) (layer F.Cu) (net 5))
 (via (at 147.32 96.52) (size 0.8) (drill 0.4) (layers F.Cu B.Cu) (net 5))
 (segment (start 147.32 96.52) (end 147.32 83.82) (width 0.25) (layer B.Cu) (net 5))
 (segment (start 147.32 83.82) (end 147.32 83.82) (width 0.25) (layer B.Cu) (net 5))
 (via (at 147.32 83.82) (size 0.8) (drill 0.4) (layers F.Cu B.Cu) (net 5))
 (segment (start 147.32 83.82) (end 149.86 83.82) (width 0.25) (layer F.Cu) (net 5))
 (segment (start 175.26 96.52) (end 177.8 96.52) (width 0.25) (layer F.Cu) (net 5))
 (segment (start 177.8 96.52) (end 177.8 96.52) (width 0.25) (layer F.Cu) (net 5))
 (via (at 177.8 96.52) (size 0.8) (drill 0.4) (layers F.Cu B.Cu) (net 5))
 (segment (start 177.8 96.52) (end 177.8 86.36) (width 0.25) (layer B.Cu) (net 5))
 (segment (start 177.8 86.36) (end 177.8 86.36) (width 0.25) (layer B.Cu) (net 5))
 (via (at 177.8 86.36) (size 0.8) (drill 0.4) (layers F.Cu B.Cu) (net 5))
 (segment (start 177.8 86.36) (end 172.72 86.36) (width 0.25) (layer F.Cu) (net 5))
 (segment (start 134.62 91.44) (end 137.16 91.44) (width 0.25) (layer F.Cu) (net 6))
 (segment (start 172.72 91.44) (end 157.48 91.44) (width 0.25) (layer F.Cu) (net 6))
 (segment (start 157.48 86.36) (end 162.56 86.36) (width 0.25) (layer F.Cu) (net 6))
 (segment (start 162.56 86.36) (end 162.56 86.36) (width 0.25) (layer F.Cu) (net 6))
 (via (at 162.56 86.36) (size 0.8) (drill 0.4) (layers F.Cu B.Cu) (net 6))
 (segment (start 162.56 86.36) (end 162.56 91.44) (width 0.25) (layer B.Cu) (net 6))
 (segment (start 162.56 91.44) (end 162.56 91.44) (width 0.25) (layer B.Cu) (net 6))
 (via (at 162.56 91.44) (size 0.8) (drill 0.4) (layers F.Cu B.Cu) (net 6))
 (segment (start 172.72 91.44) (end 175.26 91.44) (width 0.25) (layer F.Cu) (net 6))
 (segment (start 175.26 91.44) (end 175.26 91.44) (width 0.25) (layer F.Cu) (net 6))
 (via (at 175.26 91.44) (size 0.8) (drill 0.4) (layers F.Cu B.Cu) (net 6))
 (segment (start 137.16 91.44) (end 157.48 91.44) (width 0.25) (layer F.Cu) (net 6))
 (segment (start 175.26 91.44) (end 175.26 88.9) (width 0.25) (layer B.Cu) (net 6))
 (segment (start 175.26 88.9) (end 175.26 88.9) (width 0.25) (layer B.Cu) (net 6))
 (via (at 175.26 88.9) (size 0.8) (drill 0.4) (layers F.Cu B.Cu) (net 6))
 (segment (start 175.26 88.9) (end 172.72 88.9) (width 0.25) (layer F.Cu) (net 6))
 (segment (start 132.08 96.52) (end 127 96.52) (width 0.25) (layer F.Cu) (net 7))
 (segment (start 127 81.28) (end 127 81.28) (width 0.25) (layer F.Cu) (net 7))
 (segment (start 127 96.52) (end 127 96.52) (width 0.25) (layer F.Cu) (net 7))
 (via (at 127 96.52) (size 0.8) (drill 0.4) (layers F.Cu B.Cu) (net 7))
 (segment (start 127 81.28) (end 149.86 81.28) (width 0.25) (layer F.Cu) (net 7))
 (via (at 127 81.28) (size 0.8) (drill 0.4) (layers F.Cu B.Cu) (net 7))
 (segment (start 127 81.28) (end 127 96.52) (width 0.25) (layer B.Cu) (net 7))
 (segment (start 149.86 78.74) (end 147.32 78.74) (width 0.25) (layer F.Cu) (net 9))
 (segment (start 157.48 83.82) (end 167.64 83.82) (width 0.25) (layer F.Cu) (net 4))
 (segment (start 132.08 93.98) (end 129.54 93.98) (width 0.25) (layer F.Cu) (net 4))
 (segment (start 129.54 88.9) (end 129.54 88.9) (width 0.25) (layer F.Cu) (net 4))
 (segment (start 167.64 88.9) (end 167.64 88.9) (width 0.25) (layer F.Cu) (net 4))
 (via (at 167.64 88.9) (size 0.8) (drill 0.4) (layers F.Cu B.Cu) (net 4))
 (segment (start 167.64 88.9) (end 167.64 83.82) (width 0.25) (layer B.Cu) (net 4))
 (segment (start 167.64 83.82) (end 167.64 83.82) (width 0.25) (layer B.Cu) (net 4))
 (segment (start 129.54 93.98) (end 129.54 93.98) (width 0.25) (layer F.Cu) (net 4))
 (via (at 129.54 93.98) (size 0.8) (drill 0.4) (layers F.Cu B.Cu) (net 4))
 (segment (start 129.54 88.9) (end 167.64 88.9) (width 0.25) (layer F.Cu) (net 4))
 (via (at 129.54 88.9) (size 0.8) (drill 0.4) (layers F.Cu B.Cu) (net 4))
 (segment (start 129.54 93.98) (end 129.54 88.9) (width 0.25) (layer B.Cu) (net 4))
 (via (at 167.64 83.82) (size 0.8) (drill 0.4) (layers F.Cu B.Cu) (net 4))
 (segment (start 167.64 83.82) (end 172.72 83.82) (width 0.25) (layer F.Cu) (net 4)))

